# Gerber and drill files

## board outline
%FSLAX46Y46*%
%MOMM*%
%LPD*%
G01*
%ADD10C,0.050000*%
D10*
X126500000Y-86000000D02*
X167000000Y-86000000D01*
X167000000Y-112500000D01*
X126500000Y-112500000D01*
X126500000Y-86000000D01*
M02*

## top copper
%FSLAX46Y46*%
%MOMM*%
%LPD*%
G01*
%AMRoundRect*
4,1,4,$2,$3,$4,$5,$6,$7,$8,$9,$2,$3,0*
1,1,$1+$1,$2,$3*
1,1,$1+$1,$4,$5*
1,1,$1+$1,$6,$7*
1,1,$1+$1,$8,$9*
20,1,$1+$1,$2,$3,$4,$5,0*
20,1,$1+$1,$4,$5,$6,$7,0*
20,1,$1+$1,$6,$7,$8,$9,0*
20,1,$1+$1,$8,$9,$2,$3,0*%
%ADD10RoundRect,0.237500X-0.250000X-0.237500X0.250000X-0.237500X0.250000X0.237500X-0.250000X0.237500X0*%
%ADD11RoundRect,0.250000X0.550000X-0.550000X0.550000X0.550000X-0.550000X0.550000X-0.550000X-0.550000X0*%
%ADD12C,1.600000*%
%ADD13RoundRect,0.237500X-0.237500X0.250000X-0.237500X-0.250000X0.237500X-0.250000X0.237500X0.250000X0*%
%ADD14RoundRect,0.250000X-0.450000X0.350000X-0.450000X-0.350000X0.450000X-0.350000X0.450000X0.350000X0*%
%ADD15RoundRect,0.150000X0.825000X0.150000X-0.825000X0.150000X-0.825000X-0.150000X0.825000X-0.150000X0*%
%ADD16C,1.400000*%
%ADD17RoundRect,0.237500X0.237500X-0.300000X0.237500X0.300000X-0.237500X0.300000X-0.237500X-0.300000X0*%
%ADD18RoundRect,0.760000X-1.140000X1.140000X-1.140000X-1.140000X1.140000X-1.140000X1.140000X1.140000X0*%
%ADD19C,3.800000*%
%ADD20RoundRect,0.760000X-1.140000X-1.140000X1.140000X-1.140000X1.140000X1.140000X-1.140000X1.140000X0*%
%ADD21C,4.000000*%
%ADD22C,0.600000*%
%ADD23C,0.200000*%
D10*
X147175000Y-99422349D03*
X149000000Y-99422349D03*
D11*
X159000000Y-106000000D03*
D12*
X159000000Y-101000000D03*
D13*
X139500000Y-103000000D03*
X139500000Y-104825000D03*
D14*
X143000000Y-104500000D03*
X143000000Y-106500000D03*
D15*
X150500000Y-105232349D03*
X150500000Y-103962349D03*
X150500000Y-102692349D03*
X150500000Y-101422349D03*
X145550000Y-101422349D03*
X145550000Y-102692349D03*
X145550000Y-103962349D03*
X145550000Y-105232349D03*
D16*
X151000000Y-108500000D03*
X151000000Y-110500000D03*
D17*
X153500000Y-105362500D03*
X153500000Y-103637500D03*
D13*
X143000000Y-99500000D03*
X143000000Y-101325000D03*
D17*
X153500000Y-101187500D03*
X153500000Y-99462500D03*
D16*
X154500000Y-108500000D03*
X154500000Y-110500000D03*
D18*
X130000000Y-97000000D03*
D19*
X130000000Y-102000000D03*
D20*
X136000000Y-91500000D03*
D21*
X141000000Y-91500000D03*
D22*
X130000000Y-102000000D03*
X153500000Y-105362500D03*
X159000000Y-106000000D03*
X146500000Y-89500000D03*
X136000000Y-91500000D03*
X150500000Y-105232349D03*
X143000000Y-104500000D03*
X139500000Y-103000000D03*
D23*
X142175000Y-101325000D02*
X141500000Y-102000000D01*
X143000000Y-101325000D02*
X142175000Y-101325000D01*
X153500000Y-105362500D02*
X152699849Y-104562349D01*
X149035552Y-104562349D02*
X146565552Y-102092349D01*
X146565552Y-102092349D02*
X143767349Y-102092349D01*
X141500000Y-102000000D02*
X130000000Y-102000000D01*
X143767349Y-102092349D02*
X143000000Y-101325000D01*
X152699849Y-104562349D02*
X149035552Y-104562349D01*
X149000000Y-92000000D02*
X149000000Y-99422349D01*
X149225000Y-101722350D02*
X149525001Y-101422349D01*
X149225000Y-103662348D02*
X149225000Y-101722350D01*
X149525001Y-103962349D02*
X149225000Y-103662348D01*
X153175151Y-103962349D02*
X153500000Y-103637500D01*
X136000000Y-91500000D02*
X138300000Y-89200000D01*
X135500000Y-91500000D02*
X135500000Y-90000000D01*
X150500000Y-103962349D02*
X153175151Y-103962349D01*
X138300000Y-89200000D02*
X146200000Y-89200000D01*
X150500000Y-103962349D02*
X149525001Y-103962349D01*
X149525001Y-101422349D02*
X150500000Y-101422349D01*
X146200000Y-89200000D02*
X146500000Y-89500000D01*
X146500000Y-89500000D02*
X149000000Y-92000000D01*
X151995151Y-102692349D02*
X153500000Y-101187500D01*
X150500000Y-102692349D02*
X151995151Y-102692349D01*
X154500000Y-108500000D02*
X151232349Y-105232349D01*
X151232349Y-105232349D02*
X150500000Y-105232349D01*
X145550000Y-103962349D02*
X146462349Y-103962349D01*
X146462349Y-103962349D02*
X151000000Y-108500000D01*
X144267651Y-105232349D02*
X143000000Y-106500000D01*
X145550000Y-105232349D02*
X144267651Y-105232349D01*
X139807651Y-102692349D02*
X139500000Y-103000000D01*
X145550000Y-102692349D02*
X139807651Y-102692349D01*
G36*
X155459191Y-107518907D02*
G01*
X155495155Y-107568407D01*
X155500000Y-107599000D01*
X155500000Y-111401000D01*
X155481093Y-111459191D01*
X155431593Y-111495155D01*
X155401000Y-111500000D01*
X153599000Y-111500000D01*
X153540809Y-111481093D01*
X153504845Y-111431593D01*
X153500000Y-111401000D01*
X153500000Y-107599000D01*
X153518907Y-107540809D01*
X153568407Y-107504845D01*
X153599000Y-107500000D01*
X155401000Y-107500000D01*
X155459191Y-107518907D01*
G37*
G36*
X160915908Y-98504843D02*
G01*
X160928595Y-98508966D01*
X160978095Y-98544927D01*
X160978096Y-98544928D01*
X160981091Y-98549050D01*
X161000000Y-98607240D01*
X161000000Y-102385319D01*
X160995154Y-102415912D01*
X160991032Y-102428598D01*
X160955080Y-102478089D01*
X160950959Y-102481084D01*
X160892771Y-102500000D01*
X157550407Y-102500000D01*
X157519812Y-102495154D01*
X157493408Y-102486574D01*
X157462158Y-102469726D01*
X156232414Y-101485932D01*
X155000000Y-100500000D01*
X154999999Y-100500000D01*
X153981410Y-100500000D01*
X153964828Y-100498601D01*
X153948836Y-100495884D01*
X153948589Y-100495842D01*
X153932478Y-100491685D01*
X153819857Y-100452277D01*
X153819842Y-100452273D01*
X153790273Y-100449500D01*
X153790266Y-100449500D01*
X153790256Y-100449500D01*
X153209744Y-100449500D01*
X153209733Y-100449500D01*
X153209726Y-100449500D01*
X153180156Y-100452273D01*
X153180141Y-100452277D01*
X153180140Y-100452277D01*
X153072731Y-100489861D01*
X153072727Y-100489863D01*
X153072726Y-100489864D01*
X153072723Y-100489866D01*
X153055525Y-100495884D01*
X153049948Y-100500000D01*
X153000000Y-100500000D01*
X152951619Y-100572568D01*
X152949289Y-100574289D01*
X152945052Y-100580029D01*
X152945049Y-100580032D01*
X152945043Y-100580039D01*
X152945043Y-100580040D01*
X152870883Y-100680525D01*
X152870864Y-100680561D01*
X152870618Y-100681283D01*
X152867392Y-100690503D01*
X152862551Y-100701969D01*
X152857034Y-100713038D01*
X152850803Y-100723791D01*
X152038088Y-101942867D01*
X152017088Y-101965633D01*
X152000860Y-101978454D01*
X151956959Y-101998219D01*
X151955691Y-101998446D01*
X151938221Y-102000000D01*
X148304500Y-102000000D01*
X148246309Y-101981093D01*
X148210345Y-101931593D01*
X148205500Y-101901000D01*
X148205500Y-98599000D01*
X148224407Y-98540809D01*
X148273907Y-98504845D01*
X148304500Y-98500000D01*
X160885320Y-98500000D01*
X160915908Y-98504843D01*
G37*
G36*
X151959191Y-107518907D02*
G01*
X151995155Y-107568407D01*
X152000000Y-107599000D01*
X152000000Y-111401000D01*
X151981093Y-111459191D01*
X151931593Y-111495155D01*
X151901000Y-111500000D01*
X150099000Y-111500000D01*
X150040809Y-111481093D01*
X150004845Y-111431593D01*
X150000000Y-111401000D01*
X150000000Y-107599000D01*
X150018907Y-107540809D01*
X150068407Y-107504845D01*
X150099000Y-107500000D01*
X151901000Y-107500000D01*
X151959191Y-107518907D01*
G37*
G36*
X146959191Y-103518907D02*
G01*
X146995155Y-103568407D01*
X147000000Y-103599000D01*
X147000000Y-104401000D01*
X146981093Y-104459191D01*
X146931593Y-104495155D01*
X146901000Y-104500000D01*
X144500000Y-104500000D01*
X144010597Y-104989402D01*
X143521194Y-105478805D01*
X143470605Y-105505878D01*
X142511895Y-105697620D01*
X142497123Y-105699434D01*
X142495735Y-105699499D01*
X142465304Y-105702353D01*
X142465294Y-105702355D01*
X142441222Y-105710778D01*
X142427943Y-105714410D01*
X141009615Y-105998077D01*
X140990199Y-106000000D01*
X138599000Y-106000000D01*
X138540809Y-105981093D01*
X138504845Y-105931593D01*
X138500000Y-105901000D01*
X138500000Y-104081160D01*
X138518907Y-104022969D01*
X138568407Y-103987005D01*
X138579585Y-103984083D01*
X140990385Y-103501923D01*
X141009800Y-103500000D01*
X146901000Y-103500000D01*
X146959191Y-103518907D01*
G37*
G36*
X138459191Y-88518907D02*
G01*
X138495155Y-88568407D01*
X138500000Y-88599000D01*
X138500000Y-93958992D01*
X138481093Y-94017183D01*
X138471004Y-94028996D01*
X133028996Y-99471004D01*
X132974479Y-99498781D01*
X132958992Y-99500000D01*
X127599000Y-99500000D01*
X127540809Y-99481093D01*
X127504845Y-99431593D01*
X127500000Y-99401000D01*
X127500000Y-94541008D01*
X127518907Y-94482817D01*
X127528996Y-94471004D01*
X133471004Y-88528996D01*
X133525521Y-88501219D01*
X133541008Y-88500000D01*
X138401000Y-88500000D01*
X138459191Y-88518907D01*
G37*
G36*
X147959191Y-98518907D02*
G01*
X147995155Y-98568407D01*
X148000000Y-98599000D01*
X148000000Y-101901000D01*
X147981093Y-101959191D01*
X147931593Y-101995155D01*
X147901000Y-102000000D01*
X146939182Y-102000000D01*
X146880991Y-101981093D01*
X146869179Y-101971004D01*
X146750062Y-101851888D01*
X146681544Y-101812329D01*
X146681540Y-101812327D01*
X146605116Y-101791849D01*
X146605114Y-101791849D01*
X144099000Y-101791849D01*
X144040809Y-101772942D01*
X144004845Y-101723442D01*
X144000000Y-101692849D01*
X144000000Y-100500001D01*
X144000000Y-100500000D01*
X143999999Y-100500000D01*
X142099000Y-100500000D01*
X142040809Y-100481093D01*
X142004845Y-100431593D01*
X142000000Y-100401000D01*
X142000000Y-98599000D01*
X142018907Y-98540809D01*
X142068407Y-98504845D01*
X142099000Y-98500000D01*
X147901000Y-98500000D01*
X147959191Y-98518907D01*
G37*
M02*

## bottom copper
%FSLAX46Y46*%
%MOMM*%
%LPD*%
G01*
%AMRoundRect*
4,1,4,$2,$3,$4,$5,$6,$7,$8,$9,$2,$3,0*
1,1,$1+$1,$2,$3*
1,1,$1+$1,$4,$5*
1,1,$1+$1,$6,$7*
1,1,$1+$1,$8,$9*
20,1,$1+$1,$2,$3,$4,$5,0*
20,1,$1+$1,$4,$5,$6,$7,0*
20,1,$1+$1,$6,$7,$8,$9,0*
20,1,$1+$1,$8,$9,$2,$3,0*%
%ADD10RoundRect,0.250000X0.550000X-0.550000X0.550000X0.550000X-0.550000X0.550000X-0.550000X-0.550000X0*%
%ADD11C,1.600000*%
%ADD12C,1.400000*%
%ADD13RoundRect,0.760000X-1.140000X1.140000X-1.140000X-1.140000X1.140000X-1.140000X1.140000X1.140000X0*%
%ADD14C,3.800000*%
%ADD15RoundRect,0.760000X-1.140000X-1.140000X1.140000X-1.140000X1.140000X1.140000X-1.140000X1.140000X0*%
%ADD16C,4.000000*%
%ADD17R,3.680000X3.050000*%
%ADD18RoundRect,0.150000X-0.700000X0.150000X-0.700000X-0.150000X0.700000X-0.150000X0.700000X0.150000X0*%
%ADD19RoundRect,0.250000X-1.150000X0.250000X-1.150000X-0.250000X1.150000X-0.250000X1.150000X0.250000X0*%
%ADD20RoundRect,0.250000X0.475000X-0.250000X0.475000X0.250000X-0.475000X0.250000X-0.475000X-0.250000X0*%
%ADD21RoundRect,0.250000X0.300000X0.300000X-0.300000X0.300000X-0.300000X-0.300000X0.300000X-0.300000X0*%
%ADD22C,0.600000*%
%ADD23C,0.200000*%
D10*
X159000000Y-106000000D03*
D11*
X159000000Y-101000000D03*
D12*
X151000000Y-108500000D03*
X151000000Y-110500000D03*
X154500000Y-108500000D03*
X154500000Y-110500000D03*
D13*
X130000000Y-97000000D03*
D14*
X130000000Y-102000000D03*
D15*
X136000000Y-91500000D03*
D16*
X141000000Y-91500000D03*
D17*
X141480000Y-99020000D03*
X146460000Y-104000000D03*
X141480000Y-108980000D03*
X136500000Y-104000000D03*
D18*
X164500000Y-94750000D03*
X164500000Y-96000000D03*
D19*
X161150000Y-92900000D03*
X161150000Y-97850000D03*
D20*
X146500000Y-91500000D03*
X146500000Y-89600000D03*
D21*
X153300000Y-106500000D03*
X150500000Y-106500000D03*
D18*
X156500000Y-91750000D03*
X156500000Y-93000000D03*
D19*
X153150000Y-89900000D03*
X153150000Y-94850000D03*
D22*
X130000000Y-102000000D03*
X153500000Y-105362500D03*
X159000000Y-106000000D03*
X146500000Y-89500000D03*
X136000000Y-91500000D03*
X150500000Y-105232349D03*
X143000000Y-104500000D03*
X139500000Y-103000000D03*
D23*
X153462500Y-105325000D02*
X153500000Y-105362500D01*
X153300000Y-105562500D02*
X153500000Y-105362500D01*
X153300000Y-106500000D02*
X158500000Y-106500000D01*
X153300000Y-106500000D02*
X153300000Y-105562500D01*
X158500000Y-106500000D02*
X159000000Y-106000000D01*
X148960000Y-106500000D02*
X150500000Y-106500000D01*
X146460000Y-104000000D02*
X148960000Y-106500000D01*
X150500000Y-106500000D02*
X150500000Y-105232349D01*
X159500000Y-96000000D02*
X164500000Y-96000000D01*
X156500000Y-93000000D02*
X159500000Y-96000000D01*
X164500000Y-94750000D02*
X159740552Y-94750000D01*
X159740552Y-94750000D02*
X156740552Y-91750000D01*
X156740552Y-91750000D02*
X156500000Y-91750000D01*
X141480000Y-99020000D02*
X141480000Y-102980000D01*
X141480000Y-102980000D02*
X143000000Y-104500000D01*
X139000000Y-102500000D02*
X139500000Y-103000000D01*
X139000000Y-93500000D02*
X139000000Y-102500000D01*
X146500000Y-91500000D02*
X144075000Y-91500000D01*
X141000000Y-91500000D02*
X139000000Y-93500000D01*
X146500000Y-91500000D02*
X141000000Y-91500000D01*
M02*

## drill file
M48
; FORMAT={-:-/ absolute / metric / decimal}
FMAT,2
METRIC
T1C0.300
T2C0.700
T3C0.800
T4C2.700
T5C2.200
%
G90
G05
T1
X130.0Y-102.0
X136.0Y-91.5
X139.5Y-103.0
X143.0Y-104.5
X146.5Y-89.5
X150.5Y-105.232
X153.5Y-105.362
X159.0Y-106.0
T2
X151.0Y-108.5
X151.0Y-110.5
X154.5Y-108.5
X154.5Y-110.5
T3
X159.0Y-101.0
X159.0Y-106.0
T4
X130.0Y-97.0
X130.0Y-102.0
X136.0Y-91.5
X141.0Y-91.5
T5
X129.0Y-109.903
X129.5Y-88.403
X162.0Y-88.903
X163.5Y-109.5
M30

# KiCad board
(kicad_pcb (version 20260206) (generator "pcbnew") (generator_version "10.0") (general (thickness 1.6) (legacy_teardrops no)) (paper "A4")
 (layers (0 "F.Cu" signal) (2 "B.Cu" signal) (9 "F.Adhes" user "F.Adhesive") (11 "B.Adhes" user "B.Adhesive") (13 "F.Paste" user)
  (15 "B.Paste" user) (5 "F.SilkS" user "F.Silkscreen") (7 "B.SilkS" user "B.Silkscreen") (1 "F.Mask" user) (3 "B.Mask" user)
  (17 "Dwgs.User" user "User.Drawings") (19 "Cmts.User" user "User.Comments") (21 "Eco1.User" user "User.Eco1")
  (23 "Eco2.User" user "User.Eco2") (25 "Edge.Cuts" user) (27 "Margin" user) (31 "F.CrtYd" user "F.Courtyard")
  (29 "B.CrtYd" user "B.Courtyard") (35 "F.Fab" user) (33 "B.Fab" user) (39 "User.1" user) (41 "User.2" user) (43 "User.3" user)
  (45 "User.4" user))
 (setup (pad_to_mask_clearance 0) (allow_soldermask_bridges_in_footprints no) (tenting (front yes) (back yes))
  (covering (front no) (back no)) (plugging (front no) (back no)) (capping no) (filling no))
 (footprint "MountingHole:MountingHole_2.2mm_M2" (layer "F.Cu") (at 129 109.902651)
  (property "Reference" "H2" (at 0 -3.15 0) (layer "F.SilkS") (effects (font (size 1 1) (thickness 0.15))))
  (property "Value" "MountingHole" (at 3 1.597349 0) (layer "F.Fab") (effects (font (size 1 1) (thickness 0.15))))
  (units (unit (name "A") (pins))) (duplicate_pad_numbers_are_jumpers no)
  (pad "" np_thru_hole circle (at 0 0) (size 2.2 2.2) (drill 2.2) (layers "*.Cu" "*.Mask")))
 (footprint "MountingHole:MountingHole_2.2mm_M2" (layer "F.Cu") (at 163.5 109.5)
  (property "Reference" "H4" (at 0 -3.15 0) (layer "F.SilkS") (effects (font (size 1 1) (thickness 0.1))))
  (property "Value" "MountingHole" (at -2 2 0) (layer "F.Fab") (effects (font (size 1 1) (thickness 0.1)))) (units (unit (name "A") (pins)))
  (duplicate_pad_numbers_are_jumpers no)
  (pad "" np_thru_hole circle (at 0 0) (size 2.2 2.2) (drill 2.2) (layers "*.Cu" "*.Mask")))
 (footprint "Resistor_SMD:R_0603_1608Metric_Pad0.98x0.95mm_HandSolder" (layer "F.Cu") (at 148.0875 99.422349)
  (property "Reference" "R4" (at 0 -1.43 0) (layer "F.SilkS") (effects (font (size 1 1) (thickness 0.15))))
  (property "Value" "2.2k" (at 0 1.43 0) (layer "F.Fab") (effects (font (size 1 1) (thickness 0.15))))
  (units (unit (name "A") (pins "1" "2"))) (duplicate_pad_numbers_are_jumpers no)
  (pad "1" smd roundrect (at -0.9125 0) (size 0.975 0.95) (layers "F.Cu" "F.Mask" "F.Paste") (roundrect_rratio 0.25) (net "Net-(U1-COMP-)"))
  (pad "2" smd roundrect (at 0.9125 0) (size 0.975 0.95) (layers "F.Cu" "F.Mask" "F.Paste") (roundrect_rratio 0.25) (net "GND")))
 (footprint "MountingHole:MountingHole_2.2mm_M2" (layer "F.Cu") (at 162 88.902651)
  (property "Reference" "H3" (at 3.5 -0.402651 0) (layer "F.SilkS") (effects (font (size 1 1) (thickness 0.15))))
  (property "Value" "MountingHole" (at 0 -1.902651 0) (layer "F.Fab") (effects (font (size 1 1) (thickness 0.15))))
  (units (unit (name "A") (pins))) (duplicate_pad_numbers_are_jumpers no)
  (pad "" np_thru_hole circle (at 0 0) (size 2.2 2.2) (drill 2.2) (layers "*.Cu" "*.Mask")))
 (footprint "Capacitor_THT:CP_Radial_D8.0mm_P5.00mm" (layer "F.Cu") (at 159 106 90)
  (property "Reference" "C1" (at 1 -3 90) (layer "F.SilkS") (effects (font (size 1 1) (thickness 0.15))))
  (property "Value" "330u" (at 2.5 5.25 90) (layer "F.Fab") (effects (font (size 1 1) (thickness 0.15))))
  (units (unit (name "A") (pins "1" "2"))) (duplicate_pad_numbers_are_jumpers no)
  (pad "1" thru_hole roundrect (at 0 0 90) (size 1.6 1.6) (drill 0.8) (layers "*.Cu" "*.Mask") (remove_unused_layers no)
   (roundrect_rratio 0.15625) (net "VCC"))
  (pad "2" thru_hole circle (at 5 0 90) (size 1.6 1.6) (drill 0.8) (layers "*.Cu" "*.Mask") (remove_unused_layers no) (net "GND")))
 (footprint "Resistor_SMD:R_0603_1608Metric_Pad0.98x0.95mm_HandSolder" (layer "F.Cu") (at 139.5 103.9125 -90)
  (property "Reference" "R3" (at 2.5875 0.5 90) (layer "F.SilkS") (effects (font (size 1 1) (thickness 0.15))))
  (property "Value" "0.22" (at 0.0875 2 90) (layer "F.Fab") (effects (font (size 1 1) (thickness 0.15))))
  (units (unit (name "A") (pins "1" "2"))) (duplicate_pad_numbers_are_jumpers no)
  (pad "1" smd roundrect (at -0.9125 0 270) (size 0.975 0.95) (layers "F.Cu" "F.Mask" "F.Paste") (roundrect_rratio 0.25) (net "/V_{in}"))
  (pad "2" smd roundrect (at 0.9125 0 270) (size 0.975 0.95) (layers "F.Cu" "F.Mask" "F.Paste") (roundrect_rratio 0.25)
   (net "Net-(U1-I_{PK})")))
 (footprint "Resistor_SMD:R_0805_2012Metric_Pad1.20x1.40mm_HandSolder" (layer "F.Cu") (at 143 105.5 -90)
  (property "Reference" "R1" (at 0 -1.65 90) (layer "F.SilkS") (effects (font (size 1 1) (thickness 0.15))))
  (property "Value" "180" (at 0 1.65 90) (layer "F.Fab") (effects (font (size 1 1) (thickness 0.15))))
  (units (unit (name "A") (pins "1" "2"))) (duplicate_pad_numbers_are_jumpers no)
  (pad "1" smd roundrect (at -1 0 270) (size 1.2 1.4) (layers "F.Cu" "F.Mask" "F.Paste") (roundrect_rratio 0.208333) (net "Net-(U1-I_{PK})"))
  (pad "2" smd roundrect (at 1 0 270) (size 1.2 1.4) (layers "F.Cu" "F.Mask" "F.Paste") (roundrect_rratio 0.208333) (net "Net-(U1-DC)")))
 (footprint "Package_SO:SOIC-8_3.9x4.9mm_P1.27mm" (layer "F.Cu") (at 148.025 103.327349 180)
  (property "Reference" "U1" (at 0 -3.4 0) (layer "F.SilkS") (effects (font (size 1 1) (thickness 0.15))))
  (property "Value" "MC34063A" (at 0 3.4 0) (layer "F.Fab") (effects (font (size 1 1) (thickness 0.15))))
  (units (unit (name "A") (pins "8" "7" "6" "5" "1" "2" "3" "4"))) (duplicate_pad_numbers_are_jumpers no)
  (pad "1" smd roundrect (at -2.475 -1.905 180) (size 1.95 0.6) (layers "F.Cu" "F.Mask" "F.Paste") (roundrect_rratio 0.25)
   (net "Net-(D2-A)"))
  (pad "2" smd roundrect (at -2.475 -0.635 180) (size 1.95 0.6) (layers "F.Cu" "F.Mask" "F.Paste") (roundrect_rratio 0.25) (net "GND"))
  (pad "3" smd roundrect (at -2.475 0.635 180) (size 1.95 0.6) (layers "F.Cu" "F.Mask" "F.Paste") (roundrect_rratio 0.25)
   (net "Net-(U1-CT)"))
  (pad "4" smd roundrect (at -2.475 1.905 180) (size 1.95 0.6) (layers "F.Cu" "F.Mask" "F.Paste") (roundrect_rratio 0.25) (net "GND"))
  (pad "5" smd roundrect (at 2.475 1.905 180) (size 1.95 0.6) (layers "F.Cu" "F.Mask" "F.Paste") (roundrect_rratio 0.25)
   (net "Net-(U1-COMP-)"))
  (pad "6" smd roundrect (at 2.475 0.635 180) (size 1.95 0.6) (layers "F.Cu" "F.Mask" "F.Paste") (roundrect_rratio 0.25) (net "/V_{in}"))
  (pad "7" smd roundrect (at 2.475 -0.635 180) (size 1.95 0.6) (layers "F.Cu" "F.Mask" "F.Paste") (roundrect_rratio 0.25)
   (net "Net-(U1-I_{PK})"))
  (pad "8" smd roundrect (at 2.475 -1.905 180) (size 1.95 0.6) (layers "F.Cu" "F.Mask" "F.Paste") (roundrect_rratio 0.25)
   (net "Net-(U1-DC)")))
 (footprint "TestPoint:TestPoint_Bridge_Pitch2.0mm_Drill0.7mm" (layer "F.Cu") (at 151 108.5 -90)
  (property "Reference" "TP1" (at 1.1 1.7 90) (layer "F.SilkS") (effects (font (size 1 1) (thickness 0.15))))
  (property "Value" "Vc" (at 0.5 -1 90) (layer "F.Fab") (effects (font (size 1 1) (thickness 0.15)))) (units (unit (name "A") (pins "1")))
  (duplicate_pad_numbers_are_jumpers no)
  (pad "1" thru_hole circle (at 0 0 270) (size 1.4 1.4) (drill 0.7) (layers "*.Cu" "*.Mask") (remove_unused_layers no)
   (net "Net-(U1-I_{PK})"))
  (pad "1" thru_hole circle (at 2 0 270) (size 1.4 1.4) (drill 0.7) (layers "*.Cu" "*.Mask") (remove_unused_layers no)
   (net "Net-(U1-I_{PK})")))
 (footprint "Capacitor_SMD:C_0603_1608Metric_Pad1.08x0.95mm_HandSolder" (layer "F.Cu") (at 153.5 104.5 90)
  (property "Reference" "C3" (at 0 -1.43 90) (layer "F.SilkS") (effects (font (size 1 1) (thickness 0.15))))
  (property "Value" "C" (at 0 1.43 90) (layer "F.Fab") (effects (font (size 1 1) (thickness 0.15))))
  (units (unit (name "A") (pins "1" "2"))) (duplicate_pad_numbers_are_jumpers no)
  (pad "1" smd roundrect (at -0.8625 0 90) (size 1.075 0.95) (layers "F.Cu" "F.Mask" "F.Paste") (roundrect_rratio 0.25) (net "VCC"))
  (pad "2" smd roundrect (at 0.8625 0 90) (size 1.075 0.95) (layers "F.Cu" "F.Mask" "F.Paste") (roundrect_rratio 0.25) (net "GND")))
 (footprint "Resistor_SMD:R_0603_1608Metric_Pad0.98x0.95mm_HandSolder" (layer "F.Cu") (at 143 100.4125 -90)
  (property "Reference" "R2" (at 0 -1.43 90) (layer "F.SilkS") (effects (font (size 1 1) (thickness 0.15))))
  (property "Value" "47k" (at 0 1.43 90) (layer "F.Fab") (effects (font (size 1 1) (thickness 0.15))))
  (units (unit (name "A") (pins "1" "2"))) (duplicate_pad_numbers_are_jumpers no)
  (pad "1" smd roundrect (at -0.9125 0 270) (size 0.975 0.95) (layers "F.Cu" "F.Mask" "F.Paste") (roundrect_rratio 0.25)
   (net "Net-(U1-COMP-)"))
  (pad "2" smd roundrect (at 0.9125 0 270) (size 0.975 0.95) (layers "F.Cu" "F.Mask" "F.Paste") (roundrect_rratio 0.25) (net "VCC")))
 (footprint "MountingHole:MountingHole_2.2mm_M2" (layer "F.Cu") (at 129.5 88.402651)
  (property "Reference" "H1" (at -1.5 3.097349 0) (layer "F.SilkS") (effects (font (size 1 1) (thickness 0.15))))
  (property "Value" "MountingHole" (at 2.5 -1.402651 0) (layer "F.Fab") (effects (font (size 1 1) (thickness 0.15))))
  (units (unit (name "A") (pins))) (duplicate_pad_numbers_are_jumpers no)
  (pad "" np_thru_hole circle (at 0 0) (size 2.2 2.2) (drill 2.2) (layers "*.Cu" "*.Mask")))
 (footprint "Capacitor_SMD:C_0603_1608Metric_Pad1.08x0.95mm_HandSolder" (layer "F.Cu") (at 153.5 100.325 90)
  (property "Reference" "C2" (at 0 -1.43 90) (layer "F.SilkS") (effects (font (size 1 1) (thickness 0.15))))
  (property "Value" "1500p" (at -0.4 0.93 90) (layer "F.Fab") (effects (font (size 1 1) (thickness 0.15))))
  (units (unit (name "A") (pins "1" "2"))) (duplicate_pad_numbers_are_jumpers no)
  (pad "1" smd roundrect (at -0.8625 0 90) (size 1.075 0.95) (layers "F.Cu" "F.Mask" "F.Paste") (roundrect_rratio 0.25) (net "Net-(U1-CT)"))
  (pad "2" smd roundrect (at 0.8625 0 90) (size 1.075 0.95) (layers "F.Cu" "F.Mask" "F.Paste") (roundrect_rratio 0.25) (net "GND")))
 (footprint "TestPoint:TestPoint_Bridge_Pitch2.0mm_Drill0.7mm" (layer "F.Cu") (at 154.5 108.5 -90)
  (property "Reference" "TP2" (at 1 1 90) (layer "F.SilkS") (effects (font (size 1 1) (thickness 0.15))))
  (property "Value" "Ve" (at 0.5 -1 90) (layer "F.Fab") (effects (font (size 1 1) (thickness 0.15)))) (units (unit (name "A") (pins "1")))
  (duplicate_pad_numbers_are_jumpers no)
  (pad "1" thru_hole circle (at 0 0 270) (size 1.4 1.4) (drill 0.7) (layers "*.Cu" "*.Mask") (remove_unused_layers no) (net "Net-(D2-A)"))
  (pad "1" thru_hole circle (at 2 0 270) (size 1.4 1.4) (drill 0.7) (layers "*.Cu" "*.Mask") (remove_unused_layers no) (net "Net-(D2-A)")))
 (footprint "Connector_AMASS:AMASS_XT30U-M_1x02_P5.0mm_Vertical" (layer "F.Cu") (at 130 97 -90)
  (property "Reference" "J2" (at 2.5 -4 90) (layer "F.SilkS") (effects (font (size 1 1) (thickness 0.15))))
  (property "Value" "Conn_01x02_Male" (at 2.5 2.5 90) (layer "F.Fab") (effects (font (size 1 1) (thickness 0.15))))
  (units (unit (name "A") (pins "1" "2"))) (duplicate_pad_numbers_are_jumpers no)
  (pad "1" thru_hole roundrect (at 0 0 270) (size 3.8 3.8) (drill 2.7) (layers "*.Cu" "*.Mask") (remove_unused_layers no)
   (roundrect_rratio 0.2) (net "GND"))
  (pad "2" thru_hole circle (at 5 0 270) (size 3.8 3.8) (drill 2.7) (layers "*.Cu" "*.Mask") (remove_unused_layers no) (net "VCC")))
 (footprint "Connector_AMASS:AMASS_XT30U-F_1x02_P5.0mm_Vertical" (layer "B.Cu") (at 136 91.5)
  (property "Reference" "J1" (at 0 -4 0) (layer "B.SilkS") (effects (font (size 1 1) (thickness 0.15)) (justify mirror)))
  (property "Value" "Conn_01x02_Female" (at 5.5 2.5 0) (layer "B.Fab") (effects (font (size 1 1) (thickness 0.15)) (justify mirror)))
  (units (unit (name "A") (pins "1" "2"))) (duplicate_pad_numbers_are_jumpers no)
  (pad "1" thru_hole roundrect (at 0 0) (size 3.8 3.8) (drill 2.7) (layers "*.Cu" "*.Mask") (remove_unused_layers no) (roundrect_rratio 0.2)
   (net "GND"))
  (pad "2" thru_hole circle (at 5 0) (size 4 4) (drill 2.7) (layers "*.Cu" "*.Mask") (remove_unused_layers no) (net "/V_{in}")))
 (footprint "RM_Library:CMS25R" (layer "B.Cu") (at 141.48 104 -90)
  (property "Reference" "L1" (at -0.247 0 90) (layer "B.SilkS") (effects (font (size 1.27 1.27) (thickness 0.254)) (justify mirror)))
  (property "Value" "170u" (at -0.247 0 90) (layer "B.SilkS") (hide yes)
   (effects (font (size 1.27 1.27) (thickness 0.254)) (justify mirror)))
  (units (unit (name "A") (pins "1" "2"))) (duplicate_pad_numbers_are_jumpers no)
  (pad "1" smd rect (at -4.98 0 270) (size 3.05 3.68) (layers "B.Cu" "B.Mask" "B.Paste") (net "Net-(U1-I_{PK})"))
  (pad "2" smd rect (at 0 -4.98 270) (size 3.05 3.68) (layers "B.Cu" "B.Mask" "B.Paste") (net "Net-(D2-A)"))
  (pad "3" smd rect (at 4.98 0 270) (size 3.05 3.68) (layers "B.Cu" "B.Mask" "B.Paste"))
  (pad "4" smd rect (at 0 4.98 270) (size 3.05 3.68) (layers "B.Cu" "B.Mask" "B.Paste")))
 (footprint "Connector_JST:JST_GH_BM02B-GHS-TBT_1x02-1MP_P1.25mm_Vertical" (layer "B.Cu") (at 162.55 95.375 -90)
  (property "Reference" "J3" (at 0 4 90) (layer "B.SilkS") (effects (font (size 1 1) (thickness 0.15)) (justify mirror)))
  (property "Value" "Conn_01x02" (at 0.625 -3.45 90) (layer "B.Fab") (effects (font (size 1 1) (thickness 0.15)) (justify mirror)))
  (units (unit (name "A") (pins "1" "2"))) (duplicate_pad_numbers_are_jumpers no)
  (pad "1" smd roundrect (at -0.625 -1.95 270) (size 0.6 1.7) (layers "B.Cu" "B.Mask" "B.Paste") (roundrect_rratio 0.25) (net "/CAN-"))
  (pad "2" smd roundrect (at 0.625 -1.95 270) (size 0.6 1.7) (layers "B.Cu" "B.Mask" "B.Paste") (roundrect_rratio 0.25) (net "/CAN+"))
  (pad "MP" smd roundrect (at -2.475 1.4 270) (size 1 2.8) (layers "B.Cu" "B.Mask" "B.Paste") (roundrect_rratio 0.25))
  (pad "MP" smd roundrect (at 2.475 1.4 270) (size 1 2.8) (layers "B.Cu" "B.Mask" "B.Paste") (roundrect_rratio 0.25)))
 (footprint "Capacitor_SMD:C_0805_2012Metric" (layer "B.Cu") (at 146.5 90.55 90)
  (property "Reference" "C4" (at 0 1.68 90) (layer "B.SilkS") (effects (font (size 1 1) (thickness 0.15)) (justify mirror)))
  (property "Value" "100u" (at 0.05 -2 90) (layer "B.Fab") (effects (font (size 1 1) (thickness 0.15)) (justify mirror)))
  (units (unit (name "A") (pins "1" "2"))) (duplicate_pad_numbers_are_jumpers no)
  (pad "1" smd roundrect (at -0.95 0 90) (size 1 1.45) (layers "B.Cu" "B.Mask" "B.Paste") (roundrect_rratio 0.25) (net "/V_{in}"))
  (pad "2" smd roundrect (at 0.95 0 90) (size 1 1.45) (layers "B.Cu" "B.Mask" "B.Paste") (roundrect_rratio 0.25) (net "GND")))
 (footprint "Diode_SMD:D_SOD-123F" (layer "B.Cu") (at 151.9 106.5 180)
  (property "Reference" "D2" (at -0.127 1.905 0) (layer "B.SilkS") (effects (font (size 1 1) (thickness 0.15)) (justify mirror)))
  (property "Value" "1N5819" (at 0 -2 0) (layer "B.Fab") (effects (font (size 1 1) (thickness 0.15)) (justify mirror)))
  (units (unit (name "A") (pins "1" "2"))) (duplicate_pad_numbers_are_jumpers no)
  (pad "1" smd roundrect (at -1.4 0 180) (size 1.1 1.1) (layers "B.Cu" "B.Mask" "B.Paste") (roundrect_rratio 0.2272727273) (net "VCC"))
  (pad "2" smd roundrect (at 1.4 0 180) (size 1.1 1.1) (layers "B.Cu" "B.Mask" "B.Paste") (roundrect_rratio 0.2272727273) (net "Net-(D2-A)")))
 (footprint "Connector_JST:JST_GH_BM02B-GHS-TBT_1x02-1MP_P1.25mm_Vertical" (layer "B.Cu") (at 154.55 92.375 -90)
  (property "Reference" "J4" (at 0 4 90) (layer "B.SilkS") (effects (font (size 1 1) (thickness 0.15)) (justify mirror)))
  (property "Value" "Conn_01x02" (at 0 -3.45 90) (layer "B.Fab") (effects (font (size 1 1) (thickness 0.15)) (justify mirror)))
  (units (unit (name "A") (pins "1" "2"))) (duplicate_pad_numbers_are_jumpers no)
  (pad "1" smd roundrect (at -0.625 -1.95 270) (size 0.6 1.7) (layers "B.Cu" "B.Mask" "B.Paste") (roundrect_rratio 0.25) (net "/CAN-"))
  (pad "2" smd roundrect (at 0.625 -1.95 270) (size 0.6 1.7) (layers "B.Cu" "B.Mask" "B.Paste") (roundrect_rratio 0.25) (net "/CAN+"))
  (pad "MP" smd roundrect (at -2.475 1.4 270) (size 1 2.8) (layers "B.Cu" "B.Mask" "B.Paste") (roundrect_rratio 0.25))
  (pad "MP" smd roundrect (at 2.475 1.4 270) (size 1 2.8) (layers "B.Cu" "B.Mask" "B.Paste") (roundrect_rratio 0.25)))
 (gr_rect (start 126.5 86) (end 167 112.5) (stroke (width 0.05) (type default)) (fill no) (layer "Edge.Cuts"))
 (segment (start 142.175 101.325) (end 141.5 102) (width 0.2) (layer "F.Cu") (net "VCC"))
 (segment (start 143 101.325) (end 142.175 101.325) (width 0.2) (layer "F.Cu") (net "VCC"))
 (segment (start 153.5 105.3625) (end 152.699849 104.562349) (width 0.2) (layer "F.Cu") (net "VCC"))
 (segment (start 149.035552 104.562349) (end 146.565552 102.092349) (width 0.2) (layer "F.Cu") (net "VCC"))
 (segment (start 146.565552 102.092349) (end 143.767349 102.092349) (width 0.2) (layer "F.Cu") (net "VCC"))
 (segment (start 141.5 102) (end 130 102) (width 0.2) (layer "F.Cu") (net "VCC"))
 (segment (start 143.767349 102.092349) (end 143 101.325) (width 0.2) (layer "F.Cu") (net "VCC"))
 (segment (start 152.699849 104.562349) (end 149.035552 104.562349) (width 0.2) (layer "F.Cu") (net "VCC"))
 (via (at 130 102) (size 0.6) (drill 0.3) (layers "F.Cu" "B.Cu") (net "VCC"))
 (via (at 153.5 105.3625) (size 0.6) (drill 0.3) (layers "F.Cu" "B.Cu") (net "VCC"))
 (via (at 159 106) (size 0.6) (drill 0.3) (layers "F.Cu" "B.Cu") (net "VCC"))
 (segment (start 153.4625 105.325) (end 153.5 105.3625) (width 0.2) (layer "B.Cu") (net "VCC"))
 (segment (start 153.3 105.5625) (end 153.5 105.3625) (width 0.2) (layer "B.Cu") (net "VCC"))
 (segment (start 153.3 106.5) (end 158.5 106.5) (width 0.2) (layer "B.Cu") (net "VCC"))
 (segment (start 153.3 106.5) (end 153.3 105.5625) (width 0.2) (layer "B.Cu") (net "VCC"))
 (segment (start 158.5 106.5) (end 159 106) (width 0.2) (layer "B.Cu") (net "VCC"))
 (segment (start 149 92) (end 149 99.422349) (width 0.2) (layer "F.Cu") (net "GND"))
 (segment (start 149.225 101.72235) (end 149.525001 101.422349) (width 0.2) (layer "F.Cu") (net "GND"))
 (segment (start 149.225 103.662348) (end 149.225 101.72235) (width 0.2) (layer "F.Cu") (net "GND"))
 (segment (start 149.525001 103.962349) (end 149.225 103.662348) (width 0.2) (layer "F.Cu") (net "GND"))
 (segment (start 153.175151 103.962349) (end 153.5 103.6375) (width 0.2) (layer "F.Cu") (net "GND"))
 (segment (start 136 91.5) (end 138.3 89.2) (width 0.2) (layer "F.Cu") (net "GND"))
 (segment (start 135.5 91.5) (end 135.5 90) (width 0.2) (layer "F.Cu") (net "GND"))
 (segment (start 150.5 103.962349) (end 153.175151 103.962349) (width 0.2) (layer "F.Cu") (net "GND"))
 (segment (start 138.3 89.2) (end 146.2 89.2) (width 0.2) (layer "F.Cu") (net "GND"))
 (segment (start 150.5 103.962349) (end 149.525001 103.962349) (width 0.2) (layer "F.Cu") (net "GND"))
 (segment (start 149.525001 101.422349) (end 150.5 101.422349) (width 0.2) (layer "F.Cu") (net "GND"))
 (segment (start 146.2 89.2) (end 146.5 89.5) (width 0.2) (layer "F.Cu") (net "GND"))
 (segment (start 146.5 89.5) (end 149 92) (width 0.2) (layer "F.Cu") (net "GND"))
 (via (at 146.5 89.5) (size 0.6) (drill 0.3) (layers "F.Cu" "B.Cu") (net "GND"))
 (via (at 136 91.5) (size 0.6) (drill 0.3) (layers "F.Cu" "B.Cu") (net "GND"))
 (segment (start 151.995151 102.692349) (end 153.5 101.1875) (width 0.2) (layer "F.Cu") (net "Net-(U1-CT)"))
 (segment (start 150.5 102.692349) (end 151.995151 102.692349) (width 0.2) (layer "F.Cu") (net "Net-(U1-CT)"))
 (segment (start 154.5 108.5) (end 151.232349 105.232349) (width 0.2) (layer "F.Cu") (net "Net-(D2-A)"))
 (segment (start 151.232349 105.232349) (end 150.5 105.232349) (width 0.2) (layer "F.Cu") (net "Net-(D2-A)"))
 (via (at 150.5 105.232349) (size 0.6) (drill 0.3) (layers "F.Cu" "B.Cu") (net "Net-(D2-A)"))
 (segment (start 148.96 106.5) (end 150.5 106.5) (width 0.2) (layer "B.Cu") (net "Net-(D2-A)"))
 (segment (start 146.46 104) (end 148.96 106.5) (width 0.2) (layer "B.Cu") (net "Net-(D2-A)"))
 (segment (start 150.5 106.5) (end 150.5 105.232349) (width 0.2) (layer "B.Cu") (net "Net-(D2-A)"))
 (segment (start 159.5 96) (end 164.5 96) (width 0.2) (layer "B.Cu") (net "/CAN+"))
 (segment (start 156.5 93) (end 159.5 96) (width 0.2) (layer "B.Cu") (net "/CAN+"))
 (segment (start 164.5 94.75) (end 159.740552 94.75) (width 0.2) (layer "B.Cu") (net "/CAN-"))
 (segment (start 159.740552 94.75) (end 156.740552 91.75) (width 0.2) (layer "B.Cu") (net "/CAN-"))
 (segment (start 156.740552 91.75) (end 156.5 91.75) (width 0.2) (layer "B.Cu") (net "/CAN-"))
 (segment (start 145.55 103.962349) (end 146.462349 103.962349) (width 0.2) (layer "F.Cu") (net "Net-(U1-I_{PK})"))
 (segment (start 146.462349 103.962349) (end 151 108.5) (width 0.2) (layer "F.Cu") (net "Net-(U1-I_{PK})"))
 (via (at 143 104.5) (size 0.6) (drill 0.3) (layers "F.Cu" "B.Cu") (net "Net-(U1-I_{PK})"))
 (segment (start 141.48 99.02) (end 141.48 102.98) (width 0.2) (layer "B.Cu") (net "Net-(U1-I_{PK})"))
 (segment (start 141.48 102.98) (end 143 104.5) (width 0.2) (layer "B.Cu") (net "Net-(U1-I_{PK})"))
 (segment (start 144.267651 105.232349) (end 143 106.5) (width 0.2) (layer "F.Cu") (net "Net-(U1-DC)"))
 (segment (start 145.55 105.232349) (end 144.267651 105.232349) (width 0.2) (layer "F.Cu") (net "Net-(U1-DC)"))
 (segment (start 139.807651 102.692349) (end 139.5 103) (width 0.2) (layer "F.Cu") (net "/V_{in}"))
 (segment (start 145.55 102.692349) (end 139.807651 102.692349) (width 0.2) (layer "F.Cu") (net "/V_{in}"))
 (via (at 139.5 103) (size 0.6) (drill 0.3) (layers "F.Cu" "B.Cu") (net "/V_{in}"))
 (segment (start 139 102.5) (end 139.5 103) (width 0.2) (layer "B.Cu") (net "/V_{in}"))
 (segment (start 139 93.5) (end 139 102.5) (width 0.2) (layer "B.Cu") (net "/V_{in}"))
 (segment (start 146.5 91.5) (end 144.075 91.5) (width 0.2) (layer "B.Cu") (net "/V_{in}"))
 (segment (start 141 91.5) (end 139 93.5) (width 0.2) (layer "B.Cu") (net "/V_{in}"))
 (segment (start 146.5 91.5) (end 141 91.5) (width 0.2) (layer "B.Cu") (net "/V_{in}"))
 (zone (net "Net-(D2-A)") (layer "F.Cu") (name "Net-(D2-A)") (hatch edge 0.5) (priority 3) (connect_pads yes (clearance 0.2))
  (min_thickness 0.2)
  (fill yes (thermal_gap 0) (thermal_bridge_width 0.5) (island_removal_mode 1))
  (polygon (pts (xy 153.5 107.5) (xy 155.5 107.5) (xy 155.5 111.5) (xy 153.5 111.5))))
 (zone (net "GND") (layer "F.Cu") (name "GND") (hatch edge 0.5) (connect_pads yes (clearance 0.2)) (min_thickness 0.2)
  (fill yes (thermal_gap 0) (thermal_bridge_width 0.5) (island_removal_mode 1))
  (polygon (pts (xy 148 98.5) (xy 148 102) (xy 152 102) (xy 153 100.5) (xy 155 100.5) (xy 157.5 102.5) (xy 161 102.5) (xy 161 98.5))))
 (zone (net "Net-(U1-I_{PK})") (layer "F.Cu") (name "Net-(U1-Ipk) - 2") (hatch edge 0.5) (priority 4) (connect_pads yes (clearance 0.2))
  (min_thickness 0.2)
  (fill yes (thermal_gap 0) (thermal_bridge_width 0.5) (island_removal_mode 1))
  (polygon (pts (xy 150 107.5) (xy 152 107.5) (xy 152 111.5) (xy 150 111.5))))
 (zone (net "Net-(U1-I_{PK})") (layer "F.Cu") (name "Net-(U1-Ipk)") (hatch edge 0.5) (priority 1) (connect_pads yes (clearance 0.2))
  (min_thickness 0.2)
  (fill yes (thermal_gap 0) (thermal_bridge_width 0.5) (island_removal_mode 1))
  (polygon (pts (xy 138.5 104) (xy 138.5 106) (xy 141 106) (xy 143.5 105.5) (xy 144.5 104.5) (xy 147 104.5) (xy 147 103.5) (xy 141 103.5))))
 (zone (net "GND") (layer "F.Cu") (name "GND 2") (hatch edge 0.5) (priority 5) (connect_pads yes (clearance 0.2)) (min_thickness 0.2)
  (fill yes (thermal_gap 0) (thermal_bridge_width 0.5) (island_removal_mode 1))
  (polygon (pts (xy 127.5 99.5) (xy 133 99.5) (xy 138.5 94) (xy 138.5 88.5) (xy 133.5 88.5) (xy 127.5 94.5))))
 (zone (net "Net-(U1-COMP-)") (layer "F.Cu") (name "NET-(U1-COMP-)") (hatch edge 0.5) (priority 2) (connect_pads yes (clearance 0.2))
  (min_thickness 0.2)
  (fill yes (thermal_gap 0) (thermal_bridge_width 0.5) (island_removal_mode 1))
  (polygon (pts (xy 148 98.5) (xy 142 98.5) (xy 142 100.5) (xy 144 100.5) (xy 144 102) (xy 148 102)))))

